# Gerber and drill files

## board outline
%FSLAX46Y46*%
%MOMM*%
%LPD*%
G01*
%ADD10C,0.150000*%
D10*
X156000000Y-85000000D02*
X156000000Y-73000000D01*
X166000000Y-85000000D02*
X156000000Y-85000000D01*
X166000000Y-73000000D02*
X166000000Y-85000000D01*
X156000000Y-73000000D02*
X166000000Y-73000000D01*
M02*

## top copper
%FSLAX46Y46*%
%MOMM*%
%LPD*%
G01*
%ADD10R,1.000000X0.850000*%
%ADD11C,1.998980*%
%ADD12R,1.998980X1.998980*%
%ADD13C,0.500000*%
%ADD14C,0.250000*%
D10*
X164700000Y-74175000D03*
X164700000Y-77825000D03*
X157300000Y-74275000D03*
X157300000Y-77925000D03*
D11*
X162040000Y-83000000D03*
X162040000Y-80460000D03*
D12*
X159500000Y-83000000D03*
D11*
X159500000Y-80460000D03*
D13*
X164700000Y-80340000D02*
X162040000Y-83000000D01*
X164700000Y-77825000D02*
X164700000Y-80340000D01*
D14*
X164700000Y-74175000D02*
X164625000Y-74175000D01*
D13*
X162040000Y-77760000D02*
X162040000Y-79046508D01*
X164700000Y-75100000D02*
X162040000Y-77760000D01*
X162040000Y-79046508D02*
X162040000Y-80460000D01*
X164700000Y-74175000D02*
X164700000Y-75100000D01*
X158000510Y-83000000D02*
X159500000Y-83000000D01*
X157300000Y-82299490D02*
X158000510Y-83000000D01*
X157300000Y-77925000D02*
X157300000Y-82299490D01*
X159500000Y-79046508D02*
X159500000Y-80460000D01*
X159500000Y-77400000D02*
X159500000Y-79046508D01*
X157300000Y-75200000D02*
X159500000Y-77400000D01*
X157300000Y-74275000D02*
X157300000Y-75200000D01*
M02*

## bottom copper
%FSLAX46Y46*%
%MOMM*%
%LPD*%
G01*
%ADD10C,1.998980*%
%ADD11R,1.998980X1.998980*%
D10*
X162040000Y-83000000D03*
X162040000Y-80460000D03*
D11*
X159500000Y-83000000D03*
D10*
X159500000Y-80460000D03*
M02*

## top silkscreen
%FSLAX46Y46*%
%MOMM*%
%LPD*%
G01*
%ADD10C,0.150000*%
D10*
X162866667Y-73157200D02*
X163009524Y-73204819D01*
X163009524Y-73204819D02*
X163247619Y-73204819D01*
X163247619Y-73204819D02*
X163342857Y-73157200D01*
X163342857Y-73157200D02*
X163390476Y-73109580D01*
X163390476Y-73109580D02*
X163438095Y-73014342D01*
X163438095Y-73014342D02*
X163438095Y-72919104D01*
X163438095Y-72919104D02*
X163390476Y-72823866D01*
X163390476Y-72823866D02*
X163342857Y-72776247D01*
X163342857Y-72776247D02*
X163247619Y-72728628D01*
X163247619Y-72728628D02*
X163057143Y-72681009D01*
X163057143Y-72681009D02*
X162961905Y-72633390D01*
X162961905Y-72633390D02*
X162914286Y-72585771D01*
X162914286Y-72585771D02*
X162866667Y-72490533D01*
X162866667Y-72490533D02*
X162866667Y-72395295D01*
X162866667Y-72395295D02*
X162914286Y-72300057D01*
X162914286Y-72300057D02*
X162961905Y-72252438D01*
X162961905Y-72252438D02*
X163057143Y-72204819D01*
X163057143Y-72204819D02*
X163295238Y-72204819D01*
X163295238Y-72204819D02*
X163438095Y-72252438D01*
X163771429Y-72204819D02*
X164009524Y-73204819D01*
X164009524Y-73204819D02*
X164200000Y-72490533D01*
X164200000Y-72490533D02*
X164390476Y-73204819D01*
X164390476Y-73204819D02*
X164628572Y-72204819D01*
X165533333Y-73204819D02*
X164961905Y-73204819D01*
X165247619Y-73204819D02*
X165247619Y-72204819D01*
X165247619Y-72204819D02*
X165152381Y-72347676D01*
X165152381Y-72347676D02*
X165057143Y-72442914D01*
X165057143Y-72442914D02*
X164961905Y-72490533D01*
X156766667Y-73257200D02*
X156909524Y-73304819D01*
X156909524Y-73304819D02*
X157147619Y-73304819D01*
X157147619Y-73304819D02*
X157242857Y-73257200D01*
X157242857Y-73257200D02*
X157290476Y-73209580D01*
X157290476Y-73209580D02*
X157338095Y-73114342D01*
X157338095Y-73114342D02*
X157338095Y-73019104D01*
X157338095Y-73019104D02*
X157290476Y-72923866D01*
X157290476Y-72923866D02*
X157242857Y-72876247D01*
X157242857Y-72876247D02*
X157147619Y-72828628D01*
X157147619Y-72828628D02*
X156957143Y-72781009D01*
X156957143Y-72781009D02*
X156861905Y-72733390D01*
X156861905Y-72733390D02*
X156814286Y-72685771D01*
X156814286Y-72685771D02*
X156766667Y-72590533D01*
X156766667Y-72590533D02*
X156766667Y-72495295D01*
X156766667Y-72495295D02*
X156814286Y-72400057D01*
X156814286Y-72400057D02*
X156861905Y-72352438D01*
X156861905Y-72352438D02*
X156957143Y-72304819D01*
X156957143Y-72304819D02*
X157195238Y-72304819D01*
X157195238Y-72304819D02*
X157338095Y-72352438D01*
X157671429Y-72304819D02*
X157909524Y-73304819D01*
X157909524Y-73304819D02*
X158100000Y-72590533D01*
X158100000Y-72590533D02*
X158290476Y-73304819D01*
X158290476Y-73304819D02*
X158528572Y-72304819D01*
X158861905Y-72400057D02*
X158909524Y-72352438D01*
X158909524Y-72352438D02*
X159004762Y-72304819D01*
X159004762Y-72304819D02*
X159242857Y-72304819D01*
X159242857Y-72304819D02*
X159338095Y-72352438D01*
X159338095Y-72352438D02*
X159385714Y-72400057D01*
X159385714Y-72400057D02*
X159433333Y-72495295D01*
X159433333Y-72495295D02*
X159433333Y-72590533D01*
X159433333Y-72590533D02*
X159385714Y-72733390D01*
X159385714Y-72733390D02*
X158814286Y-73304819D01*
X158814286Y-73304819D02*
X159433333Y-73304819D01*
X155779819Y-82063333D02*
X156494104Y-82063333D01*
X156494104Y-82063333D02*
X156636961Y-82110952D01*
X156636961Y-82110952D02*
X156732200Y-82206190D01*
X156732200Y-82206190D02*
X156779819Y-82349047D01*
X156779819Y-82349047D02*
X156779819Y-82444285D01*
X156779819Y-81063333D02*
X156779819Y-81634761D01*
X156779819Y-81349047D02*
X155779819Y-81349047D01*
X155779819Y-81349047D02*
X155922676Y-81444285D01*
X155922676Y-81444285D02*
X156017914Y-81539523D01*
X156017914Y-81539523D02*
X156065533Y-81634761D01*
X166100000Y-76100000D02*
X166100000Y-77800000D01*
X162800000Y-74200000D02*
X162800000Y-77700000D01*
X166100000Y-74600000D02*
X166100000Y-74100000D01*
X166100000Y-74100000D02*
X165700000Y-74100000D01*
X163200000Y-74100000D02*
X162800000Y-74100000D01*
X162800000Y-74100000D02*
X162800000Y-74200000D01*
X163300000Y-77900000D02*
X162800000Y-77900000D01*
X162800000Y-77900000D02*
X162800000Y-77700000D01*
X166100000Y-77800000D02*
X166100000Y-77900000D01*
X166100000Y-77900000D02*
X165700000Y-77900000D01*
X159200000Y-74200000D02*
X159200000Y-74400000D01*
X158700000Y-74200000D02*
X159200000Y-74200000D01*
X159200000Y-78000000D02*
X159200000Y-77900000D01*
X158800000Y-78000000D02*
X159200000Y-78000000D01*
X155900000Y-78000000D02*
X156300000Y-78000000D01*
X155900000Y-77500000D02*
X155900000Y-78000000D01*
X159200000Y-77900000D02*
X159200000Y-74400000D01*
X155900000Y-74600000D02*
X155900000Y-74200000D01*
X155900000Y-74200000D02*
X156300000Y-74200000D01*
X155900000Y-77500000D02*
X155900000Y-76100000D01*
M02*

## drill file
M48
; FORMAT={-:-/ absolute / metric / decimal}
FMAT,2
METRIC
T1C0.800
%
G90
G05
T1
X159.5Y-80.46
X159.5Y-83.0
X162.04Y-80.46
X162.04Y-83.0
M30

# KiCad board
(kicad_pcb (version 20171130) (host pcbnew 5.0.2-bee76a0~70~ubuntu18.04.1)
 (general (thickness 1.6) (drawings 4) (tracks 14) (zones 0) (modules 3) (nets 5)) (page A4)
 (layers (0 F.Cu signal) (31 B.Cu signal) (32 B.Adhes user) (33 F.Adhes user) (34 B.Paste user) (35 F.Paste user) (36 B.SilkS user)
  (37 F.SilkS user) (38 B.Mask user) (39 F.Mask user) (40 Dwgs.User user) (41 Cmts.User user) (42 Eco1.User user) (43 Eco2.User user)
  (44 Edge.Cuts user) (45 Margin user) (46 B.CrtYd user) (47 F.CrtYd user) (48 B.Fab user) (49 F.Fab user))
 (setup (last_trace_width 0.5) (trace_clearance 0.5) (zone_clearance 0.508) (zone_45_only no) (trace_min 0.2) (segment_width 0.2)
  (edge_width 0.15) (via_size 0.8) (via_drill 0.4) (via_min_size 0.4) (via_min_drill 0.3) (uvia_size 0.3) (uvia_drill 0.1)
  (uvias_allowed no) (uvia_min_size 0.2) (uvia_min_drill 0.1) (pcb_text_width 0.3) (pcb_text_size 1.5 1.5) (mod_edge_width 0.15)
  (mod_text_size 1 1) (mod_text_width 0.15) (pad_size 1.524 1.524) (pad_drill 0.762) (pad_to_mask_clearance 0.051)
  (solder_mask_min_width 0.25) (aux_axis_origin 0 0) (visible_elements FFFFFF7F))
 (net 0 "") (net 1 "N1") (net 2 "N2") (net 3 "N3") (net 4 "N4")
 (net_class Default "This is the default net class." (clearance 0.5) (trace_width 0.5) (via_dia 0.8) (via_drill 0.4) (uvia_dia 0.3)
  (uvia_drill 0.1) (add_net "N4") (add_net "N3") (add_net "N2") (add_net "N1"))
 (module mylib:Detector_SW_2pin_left (layer F.Cu) (at 164.7 76 270)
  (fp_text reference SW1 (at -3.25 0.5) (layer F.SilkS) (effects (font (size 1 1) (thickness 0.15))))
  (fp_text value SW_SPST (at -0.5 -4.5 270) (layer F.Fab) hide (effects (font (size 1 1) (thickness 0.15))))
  (fp_line (start 0.1 -1.4) (end 1.8 -1.4) (layer F.SilkS) (width 0.15))
  (fp_line (start -1.8 1.9) (end 1.7 1.9) (layer F.SilkS) (width 0.15))
  (fp_line (start -1.4 -1.4) (end -1.9 -1.4) (layer F.SilkS) (width 0.15))
  (fp_line (start -1.9 -1.4) (end -1.9 -1) (layer F.SilkS) (width 0.15))
  (fp_line (start -1.9 1.5) (end -1.9 1.9) (layer F.SilkS) (width 0.15))
  (fp_line (start -1.9 1.9) (end -1.8 1.9) (layer F.SilkS) (width 0.15))
  (fp_line (start 1.9 1.4) (end 1.9 1.9) (layer F.SilkS) (width 0.15))
  (fp_line (start 1.9 1.9) (end 1.7 1.9) (layer F.SilkS) (width 0.15))
  (fp_line (start 1.8 -1.4) (end 1.9 -1.4) (layer F.SilkS) (width 0.15))
  (fp_line (start 1.9 -1.4) (end 1.9 -1) (layer F.SilkS) (width 0.15))
  (pad 1 smd rect (at -1.825 0 270) (size 0.85 1) (layers F.Cu F.Paste F.Mask) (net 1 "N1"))
  (pad 2 smd rect (at 1.825 0 270) (size 0.85 1) (layers F.Cu F.Paste F.Mask) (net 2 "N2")))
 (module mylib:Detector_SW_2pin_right (layer F.Cu) (at 157.3 76.1 90)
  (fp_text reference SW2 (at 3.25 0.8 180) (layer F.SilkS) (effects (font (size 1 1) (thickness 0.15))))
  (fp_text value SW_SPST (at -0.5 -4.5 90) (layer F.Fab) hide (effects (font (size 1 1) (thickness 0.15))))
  (fp_line (start 1.9 1.9) (end 1.7 1.9) (layer F.SilkS) (width 0.15))
  (fp_line (start 1.9 1.4) (end 1.9 1.9) (layer F.SilkS) (width 0.15))
  (fp_line (start -1.9 1.9) (end -1.8 1.9) (layer F.SilkS) (width 0.15))
  (fp_line (start -1.9 1.5) (end -1.9 1.9) (layer F.SilkS) (width 0.15))
  (fp_line (start -1.9 -1.4) (end -1.9 -1) (layer F.SilkS) (width 0.15))
  (fp_line (start -1.4 -1.4) (end -1.9 -1.4) (layer F.SilkS) (width 0.15))
  (fp_line (start -1.8 1.9) (end 1.7 1.9) (layer F.SilkS) (width 0.15))
  (fp_line (start 1.5 -1.4) (end 1.9 -1.4) (layer F.SilkS) (width 0.15))
  (fp_line (start 1.9 -1.4) (end 1.9 -1) (layer F.SilkS) (width 0.15))
  (fp_line (start -1.4 -1.4) (end 0 -1.4) (layer F.SilkS) (width 0.15))
  (pad 2 smd rect (at 1.825 0 90) (size 0.85 1) (layers F.Cu F.Paste F.Mask) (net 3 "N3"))
  (pad 1 smd rect (at -1.825 0 90) (size 0.85 1) (layers F.Cu F.Paste F.Mask) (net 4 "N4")))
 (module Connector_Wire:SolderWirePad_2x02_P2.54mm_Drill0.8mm (layer F.Cu) (at 159.5 83 90)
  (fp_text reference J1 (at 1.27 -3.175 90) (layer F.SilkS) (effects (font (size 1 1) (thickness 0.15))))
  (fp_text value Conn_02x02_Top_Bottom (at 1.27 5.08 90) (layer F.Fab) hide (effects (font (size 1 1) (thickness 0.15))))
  (pad 3 thru_hole circle (at 0 2.54 90) (size 1.99898 1.99898) (drill 0.8001) (layers *.Cu *.Mask) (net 2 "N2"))
  (pad 4 thru_hole circle (at 2.54 2.54 90) (size 1.99898 1.99898) (drill 0.8001) (layers *.Cu *.Mask) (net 1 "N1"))
  (pad 1 thru_hole rect (at 0 0 90) (size 1.99898 1.99898) (drill 0.8001) (layers *.Cu *.Mask) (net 4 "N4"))
  (pad 2 thru_hole circle (at 2.54 0 90) (size 1.99898 1.99898) (drill 0.8001) (layers *.Cu *.Mask) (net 3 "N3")))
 (gr_line (start 156 85) (end 156 73) (layer Edge.Cuts) (width 0.15))
 (gr_line (start 166 85) (end 156 85) (layer Edge.Cuts) (width 0.15))
 (gr_line (start 166 73) (end 166 85) (layer Edge.Cuts) (width 0.15))
 (gr_line (start 156 73) (end 166 73) (layer Edge.Cuts) (width 0.15))
 (segment (start 164.7 80.34) (end 162.04 83) (width 0.5) (layer F.Cu) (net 2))
 (segment (start 164.7 77.825) (end 164.7 80.34) (width 0.5) (layer F.Cu) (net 2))
 (segment (start 164.7 74.175) (end 164.625 74.175) (width 0.25) (layer F.Cu) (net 1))
 (segment (start 162.04 77.76) (end 162.04 79.046508) (width 0.5) (layer F.Cu) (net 1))
 (segment (start 164.7 75.1) (end 162.04 77.76) (width 0.5) (layer F.Cu) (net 1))
 (segment (start 162.04 79.046508) (end 162.04 80.46) (width 0.5) (layer F.Cu) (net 1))
 (segment (start 164.7 74.175) (end 164.7 75.1) (width 0.5) (layer F.Cu) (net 1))
 (segment (start 158.00051 83) (end 159.5 83) (width 0.5) (layer F.Cu) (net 4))
 (segment (start 157.3 82.29949) (end 158.00051 83) (width 0.5) (layer F.Cu) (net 4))
 (segment (start 157.3 77.925) (end 157.3 82.29949) (width 0.5) (layer F.Cu) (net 4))
 (segment (start 159.5 79.046508) (end 159.5 80.46) (width 0.5) (layer F.Cu) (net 3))
 (segment (start 159.5 77.4) (end 159.5 79.046508) (width 0.5) (layer F.Cu) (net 3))
 (segment (start 157.3 75.2) (end 159.5 77.4) (width 0.5) (layer F.Cu) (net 3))
 (segment (start 157.3 74.275) (end 157.3 75.2) (width 0.5) (layer F.Cu) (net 3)))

